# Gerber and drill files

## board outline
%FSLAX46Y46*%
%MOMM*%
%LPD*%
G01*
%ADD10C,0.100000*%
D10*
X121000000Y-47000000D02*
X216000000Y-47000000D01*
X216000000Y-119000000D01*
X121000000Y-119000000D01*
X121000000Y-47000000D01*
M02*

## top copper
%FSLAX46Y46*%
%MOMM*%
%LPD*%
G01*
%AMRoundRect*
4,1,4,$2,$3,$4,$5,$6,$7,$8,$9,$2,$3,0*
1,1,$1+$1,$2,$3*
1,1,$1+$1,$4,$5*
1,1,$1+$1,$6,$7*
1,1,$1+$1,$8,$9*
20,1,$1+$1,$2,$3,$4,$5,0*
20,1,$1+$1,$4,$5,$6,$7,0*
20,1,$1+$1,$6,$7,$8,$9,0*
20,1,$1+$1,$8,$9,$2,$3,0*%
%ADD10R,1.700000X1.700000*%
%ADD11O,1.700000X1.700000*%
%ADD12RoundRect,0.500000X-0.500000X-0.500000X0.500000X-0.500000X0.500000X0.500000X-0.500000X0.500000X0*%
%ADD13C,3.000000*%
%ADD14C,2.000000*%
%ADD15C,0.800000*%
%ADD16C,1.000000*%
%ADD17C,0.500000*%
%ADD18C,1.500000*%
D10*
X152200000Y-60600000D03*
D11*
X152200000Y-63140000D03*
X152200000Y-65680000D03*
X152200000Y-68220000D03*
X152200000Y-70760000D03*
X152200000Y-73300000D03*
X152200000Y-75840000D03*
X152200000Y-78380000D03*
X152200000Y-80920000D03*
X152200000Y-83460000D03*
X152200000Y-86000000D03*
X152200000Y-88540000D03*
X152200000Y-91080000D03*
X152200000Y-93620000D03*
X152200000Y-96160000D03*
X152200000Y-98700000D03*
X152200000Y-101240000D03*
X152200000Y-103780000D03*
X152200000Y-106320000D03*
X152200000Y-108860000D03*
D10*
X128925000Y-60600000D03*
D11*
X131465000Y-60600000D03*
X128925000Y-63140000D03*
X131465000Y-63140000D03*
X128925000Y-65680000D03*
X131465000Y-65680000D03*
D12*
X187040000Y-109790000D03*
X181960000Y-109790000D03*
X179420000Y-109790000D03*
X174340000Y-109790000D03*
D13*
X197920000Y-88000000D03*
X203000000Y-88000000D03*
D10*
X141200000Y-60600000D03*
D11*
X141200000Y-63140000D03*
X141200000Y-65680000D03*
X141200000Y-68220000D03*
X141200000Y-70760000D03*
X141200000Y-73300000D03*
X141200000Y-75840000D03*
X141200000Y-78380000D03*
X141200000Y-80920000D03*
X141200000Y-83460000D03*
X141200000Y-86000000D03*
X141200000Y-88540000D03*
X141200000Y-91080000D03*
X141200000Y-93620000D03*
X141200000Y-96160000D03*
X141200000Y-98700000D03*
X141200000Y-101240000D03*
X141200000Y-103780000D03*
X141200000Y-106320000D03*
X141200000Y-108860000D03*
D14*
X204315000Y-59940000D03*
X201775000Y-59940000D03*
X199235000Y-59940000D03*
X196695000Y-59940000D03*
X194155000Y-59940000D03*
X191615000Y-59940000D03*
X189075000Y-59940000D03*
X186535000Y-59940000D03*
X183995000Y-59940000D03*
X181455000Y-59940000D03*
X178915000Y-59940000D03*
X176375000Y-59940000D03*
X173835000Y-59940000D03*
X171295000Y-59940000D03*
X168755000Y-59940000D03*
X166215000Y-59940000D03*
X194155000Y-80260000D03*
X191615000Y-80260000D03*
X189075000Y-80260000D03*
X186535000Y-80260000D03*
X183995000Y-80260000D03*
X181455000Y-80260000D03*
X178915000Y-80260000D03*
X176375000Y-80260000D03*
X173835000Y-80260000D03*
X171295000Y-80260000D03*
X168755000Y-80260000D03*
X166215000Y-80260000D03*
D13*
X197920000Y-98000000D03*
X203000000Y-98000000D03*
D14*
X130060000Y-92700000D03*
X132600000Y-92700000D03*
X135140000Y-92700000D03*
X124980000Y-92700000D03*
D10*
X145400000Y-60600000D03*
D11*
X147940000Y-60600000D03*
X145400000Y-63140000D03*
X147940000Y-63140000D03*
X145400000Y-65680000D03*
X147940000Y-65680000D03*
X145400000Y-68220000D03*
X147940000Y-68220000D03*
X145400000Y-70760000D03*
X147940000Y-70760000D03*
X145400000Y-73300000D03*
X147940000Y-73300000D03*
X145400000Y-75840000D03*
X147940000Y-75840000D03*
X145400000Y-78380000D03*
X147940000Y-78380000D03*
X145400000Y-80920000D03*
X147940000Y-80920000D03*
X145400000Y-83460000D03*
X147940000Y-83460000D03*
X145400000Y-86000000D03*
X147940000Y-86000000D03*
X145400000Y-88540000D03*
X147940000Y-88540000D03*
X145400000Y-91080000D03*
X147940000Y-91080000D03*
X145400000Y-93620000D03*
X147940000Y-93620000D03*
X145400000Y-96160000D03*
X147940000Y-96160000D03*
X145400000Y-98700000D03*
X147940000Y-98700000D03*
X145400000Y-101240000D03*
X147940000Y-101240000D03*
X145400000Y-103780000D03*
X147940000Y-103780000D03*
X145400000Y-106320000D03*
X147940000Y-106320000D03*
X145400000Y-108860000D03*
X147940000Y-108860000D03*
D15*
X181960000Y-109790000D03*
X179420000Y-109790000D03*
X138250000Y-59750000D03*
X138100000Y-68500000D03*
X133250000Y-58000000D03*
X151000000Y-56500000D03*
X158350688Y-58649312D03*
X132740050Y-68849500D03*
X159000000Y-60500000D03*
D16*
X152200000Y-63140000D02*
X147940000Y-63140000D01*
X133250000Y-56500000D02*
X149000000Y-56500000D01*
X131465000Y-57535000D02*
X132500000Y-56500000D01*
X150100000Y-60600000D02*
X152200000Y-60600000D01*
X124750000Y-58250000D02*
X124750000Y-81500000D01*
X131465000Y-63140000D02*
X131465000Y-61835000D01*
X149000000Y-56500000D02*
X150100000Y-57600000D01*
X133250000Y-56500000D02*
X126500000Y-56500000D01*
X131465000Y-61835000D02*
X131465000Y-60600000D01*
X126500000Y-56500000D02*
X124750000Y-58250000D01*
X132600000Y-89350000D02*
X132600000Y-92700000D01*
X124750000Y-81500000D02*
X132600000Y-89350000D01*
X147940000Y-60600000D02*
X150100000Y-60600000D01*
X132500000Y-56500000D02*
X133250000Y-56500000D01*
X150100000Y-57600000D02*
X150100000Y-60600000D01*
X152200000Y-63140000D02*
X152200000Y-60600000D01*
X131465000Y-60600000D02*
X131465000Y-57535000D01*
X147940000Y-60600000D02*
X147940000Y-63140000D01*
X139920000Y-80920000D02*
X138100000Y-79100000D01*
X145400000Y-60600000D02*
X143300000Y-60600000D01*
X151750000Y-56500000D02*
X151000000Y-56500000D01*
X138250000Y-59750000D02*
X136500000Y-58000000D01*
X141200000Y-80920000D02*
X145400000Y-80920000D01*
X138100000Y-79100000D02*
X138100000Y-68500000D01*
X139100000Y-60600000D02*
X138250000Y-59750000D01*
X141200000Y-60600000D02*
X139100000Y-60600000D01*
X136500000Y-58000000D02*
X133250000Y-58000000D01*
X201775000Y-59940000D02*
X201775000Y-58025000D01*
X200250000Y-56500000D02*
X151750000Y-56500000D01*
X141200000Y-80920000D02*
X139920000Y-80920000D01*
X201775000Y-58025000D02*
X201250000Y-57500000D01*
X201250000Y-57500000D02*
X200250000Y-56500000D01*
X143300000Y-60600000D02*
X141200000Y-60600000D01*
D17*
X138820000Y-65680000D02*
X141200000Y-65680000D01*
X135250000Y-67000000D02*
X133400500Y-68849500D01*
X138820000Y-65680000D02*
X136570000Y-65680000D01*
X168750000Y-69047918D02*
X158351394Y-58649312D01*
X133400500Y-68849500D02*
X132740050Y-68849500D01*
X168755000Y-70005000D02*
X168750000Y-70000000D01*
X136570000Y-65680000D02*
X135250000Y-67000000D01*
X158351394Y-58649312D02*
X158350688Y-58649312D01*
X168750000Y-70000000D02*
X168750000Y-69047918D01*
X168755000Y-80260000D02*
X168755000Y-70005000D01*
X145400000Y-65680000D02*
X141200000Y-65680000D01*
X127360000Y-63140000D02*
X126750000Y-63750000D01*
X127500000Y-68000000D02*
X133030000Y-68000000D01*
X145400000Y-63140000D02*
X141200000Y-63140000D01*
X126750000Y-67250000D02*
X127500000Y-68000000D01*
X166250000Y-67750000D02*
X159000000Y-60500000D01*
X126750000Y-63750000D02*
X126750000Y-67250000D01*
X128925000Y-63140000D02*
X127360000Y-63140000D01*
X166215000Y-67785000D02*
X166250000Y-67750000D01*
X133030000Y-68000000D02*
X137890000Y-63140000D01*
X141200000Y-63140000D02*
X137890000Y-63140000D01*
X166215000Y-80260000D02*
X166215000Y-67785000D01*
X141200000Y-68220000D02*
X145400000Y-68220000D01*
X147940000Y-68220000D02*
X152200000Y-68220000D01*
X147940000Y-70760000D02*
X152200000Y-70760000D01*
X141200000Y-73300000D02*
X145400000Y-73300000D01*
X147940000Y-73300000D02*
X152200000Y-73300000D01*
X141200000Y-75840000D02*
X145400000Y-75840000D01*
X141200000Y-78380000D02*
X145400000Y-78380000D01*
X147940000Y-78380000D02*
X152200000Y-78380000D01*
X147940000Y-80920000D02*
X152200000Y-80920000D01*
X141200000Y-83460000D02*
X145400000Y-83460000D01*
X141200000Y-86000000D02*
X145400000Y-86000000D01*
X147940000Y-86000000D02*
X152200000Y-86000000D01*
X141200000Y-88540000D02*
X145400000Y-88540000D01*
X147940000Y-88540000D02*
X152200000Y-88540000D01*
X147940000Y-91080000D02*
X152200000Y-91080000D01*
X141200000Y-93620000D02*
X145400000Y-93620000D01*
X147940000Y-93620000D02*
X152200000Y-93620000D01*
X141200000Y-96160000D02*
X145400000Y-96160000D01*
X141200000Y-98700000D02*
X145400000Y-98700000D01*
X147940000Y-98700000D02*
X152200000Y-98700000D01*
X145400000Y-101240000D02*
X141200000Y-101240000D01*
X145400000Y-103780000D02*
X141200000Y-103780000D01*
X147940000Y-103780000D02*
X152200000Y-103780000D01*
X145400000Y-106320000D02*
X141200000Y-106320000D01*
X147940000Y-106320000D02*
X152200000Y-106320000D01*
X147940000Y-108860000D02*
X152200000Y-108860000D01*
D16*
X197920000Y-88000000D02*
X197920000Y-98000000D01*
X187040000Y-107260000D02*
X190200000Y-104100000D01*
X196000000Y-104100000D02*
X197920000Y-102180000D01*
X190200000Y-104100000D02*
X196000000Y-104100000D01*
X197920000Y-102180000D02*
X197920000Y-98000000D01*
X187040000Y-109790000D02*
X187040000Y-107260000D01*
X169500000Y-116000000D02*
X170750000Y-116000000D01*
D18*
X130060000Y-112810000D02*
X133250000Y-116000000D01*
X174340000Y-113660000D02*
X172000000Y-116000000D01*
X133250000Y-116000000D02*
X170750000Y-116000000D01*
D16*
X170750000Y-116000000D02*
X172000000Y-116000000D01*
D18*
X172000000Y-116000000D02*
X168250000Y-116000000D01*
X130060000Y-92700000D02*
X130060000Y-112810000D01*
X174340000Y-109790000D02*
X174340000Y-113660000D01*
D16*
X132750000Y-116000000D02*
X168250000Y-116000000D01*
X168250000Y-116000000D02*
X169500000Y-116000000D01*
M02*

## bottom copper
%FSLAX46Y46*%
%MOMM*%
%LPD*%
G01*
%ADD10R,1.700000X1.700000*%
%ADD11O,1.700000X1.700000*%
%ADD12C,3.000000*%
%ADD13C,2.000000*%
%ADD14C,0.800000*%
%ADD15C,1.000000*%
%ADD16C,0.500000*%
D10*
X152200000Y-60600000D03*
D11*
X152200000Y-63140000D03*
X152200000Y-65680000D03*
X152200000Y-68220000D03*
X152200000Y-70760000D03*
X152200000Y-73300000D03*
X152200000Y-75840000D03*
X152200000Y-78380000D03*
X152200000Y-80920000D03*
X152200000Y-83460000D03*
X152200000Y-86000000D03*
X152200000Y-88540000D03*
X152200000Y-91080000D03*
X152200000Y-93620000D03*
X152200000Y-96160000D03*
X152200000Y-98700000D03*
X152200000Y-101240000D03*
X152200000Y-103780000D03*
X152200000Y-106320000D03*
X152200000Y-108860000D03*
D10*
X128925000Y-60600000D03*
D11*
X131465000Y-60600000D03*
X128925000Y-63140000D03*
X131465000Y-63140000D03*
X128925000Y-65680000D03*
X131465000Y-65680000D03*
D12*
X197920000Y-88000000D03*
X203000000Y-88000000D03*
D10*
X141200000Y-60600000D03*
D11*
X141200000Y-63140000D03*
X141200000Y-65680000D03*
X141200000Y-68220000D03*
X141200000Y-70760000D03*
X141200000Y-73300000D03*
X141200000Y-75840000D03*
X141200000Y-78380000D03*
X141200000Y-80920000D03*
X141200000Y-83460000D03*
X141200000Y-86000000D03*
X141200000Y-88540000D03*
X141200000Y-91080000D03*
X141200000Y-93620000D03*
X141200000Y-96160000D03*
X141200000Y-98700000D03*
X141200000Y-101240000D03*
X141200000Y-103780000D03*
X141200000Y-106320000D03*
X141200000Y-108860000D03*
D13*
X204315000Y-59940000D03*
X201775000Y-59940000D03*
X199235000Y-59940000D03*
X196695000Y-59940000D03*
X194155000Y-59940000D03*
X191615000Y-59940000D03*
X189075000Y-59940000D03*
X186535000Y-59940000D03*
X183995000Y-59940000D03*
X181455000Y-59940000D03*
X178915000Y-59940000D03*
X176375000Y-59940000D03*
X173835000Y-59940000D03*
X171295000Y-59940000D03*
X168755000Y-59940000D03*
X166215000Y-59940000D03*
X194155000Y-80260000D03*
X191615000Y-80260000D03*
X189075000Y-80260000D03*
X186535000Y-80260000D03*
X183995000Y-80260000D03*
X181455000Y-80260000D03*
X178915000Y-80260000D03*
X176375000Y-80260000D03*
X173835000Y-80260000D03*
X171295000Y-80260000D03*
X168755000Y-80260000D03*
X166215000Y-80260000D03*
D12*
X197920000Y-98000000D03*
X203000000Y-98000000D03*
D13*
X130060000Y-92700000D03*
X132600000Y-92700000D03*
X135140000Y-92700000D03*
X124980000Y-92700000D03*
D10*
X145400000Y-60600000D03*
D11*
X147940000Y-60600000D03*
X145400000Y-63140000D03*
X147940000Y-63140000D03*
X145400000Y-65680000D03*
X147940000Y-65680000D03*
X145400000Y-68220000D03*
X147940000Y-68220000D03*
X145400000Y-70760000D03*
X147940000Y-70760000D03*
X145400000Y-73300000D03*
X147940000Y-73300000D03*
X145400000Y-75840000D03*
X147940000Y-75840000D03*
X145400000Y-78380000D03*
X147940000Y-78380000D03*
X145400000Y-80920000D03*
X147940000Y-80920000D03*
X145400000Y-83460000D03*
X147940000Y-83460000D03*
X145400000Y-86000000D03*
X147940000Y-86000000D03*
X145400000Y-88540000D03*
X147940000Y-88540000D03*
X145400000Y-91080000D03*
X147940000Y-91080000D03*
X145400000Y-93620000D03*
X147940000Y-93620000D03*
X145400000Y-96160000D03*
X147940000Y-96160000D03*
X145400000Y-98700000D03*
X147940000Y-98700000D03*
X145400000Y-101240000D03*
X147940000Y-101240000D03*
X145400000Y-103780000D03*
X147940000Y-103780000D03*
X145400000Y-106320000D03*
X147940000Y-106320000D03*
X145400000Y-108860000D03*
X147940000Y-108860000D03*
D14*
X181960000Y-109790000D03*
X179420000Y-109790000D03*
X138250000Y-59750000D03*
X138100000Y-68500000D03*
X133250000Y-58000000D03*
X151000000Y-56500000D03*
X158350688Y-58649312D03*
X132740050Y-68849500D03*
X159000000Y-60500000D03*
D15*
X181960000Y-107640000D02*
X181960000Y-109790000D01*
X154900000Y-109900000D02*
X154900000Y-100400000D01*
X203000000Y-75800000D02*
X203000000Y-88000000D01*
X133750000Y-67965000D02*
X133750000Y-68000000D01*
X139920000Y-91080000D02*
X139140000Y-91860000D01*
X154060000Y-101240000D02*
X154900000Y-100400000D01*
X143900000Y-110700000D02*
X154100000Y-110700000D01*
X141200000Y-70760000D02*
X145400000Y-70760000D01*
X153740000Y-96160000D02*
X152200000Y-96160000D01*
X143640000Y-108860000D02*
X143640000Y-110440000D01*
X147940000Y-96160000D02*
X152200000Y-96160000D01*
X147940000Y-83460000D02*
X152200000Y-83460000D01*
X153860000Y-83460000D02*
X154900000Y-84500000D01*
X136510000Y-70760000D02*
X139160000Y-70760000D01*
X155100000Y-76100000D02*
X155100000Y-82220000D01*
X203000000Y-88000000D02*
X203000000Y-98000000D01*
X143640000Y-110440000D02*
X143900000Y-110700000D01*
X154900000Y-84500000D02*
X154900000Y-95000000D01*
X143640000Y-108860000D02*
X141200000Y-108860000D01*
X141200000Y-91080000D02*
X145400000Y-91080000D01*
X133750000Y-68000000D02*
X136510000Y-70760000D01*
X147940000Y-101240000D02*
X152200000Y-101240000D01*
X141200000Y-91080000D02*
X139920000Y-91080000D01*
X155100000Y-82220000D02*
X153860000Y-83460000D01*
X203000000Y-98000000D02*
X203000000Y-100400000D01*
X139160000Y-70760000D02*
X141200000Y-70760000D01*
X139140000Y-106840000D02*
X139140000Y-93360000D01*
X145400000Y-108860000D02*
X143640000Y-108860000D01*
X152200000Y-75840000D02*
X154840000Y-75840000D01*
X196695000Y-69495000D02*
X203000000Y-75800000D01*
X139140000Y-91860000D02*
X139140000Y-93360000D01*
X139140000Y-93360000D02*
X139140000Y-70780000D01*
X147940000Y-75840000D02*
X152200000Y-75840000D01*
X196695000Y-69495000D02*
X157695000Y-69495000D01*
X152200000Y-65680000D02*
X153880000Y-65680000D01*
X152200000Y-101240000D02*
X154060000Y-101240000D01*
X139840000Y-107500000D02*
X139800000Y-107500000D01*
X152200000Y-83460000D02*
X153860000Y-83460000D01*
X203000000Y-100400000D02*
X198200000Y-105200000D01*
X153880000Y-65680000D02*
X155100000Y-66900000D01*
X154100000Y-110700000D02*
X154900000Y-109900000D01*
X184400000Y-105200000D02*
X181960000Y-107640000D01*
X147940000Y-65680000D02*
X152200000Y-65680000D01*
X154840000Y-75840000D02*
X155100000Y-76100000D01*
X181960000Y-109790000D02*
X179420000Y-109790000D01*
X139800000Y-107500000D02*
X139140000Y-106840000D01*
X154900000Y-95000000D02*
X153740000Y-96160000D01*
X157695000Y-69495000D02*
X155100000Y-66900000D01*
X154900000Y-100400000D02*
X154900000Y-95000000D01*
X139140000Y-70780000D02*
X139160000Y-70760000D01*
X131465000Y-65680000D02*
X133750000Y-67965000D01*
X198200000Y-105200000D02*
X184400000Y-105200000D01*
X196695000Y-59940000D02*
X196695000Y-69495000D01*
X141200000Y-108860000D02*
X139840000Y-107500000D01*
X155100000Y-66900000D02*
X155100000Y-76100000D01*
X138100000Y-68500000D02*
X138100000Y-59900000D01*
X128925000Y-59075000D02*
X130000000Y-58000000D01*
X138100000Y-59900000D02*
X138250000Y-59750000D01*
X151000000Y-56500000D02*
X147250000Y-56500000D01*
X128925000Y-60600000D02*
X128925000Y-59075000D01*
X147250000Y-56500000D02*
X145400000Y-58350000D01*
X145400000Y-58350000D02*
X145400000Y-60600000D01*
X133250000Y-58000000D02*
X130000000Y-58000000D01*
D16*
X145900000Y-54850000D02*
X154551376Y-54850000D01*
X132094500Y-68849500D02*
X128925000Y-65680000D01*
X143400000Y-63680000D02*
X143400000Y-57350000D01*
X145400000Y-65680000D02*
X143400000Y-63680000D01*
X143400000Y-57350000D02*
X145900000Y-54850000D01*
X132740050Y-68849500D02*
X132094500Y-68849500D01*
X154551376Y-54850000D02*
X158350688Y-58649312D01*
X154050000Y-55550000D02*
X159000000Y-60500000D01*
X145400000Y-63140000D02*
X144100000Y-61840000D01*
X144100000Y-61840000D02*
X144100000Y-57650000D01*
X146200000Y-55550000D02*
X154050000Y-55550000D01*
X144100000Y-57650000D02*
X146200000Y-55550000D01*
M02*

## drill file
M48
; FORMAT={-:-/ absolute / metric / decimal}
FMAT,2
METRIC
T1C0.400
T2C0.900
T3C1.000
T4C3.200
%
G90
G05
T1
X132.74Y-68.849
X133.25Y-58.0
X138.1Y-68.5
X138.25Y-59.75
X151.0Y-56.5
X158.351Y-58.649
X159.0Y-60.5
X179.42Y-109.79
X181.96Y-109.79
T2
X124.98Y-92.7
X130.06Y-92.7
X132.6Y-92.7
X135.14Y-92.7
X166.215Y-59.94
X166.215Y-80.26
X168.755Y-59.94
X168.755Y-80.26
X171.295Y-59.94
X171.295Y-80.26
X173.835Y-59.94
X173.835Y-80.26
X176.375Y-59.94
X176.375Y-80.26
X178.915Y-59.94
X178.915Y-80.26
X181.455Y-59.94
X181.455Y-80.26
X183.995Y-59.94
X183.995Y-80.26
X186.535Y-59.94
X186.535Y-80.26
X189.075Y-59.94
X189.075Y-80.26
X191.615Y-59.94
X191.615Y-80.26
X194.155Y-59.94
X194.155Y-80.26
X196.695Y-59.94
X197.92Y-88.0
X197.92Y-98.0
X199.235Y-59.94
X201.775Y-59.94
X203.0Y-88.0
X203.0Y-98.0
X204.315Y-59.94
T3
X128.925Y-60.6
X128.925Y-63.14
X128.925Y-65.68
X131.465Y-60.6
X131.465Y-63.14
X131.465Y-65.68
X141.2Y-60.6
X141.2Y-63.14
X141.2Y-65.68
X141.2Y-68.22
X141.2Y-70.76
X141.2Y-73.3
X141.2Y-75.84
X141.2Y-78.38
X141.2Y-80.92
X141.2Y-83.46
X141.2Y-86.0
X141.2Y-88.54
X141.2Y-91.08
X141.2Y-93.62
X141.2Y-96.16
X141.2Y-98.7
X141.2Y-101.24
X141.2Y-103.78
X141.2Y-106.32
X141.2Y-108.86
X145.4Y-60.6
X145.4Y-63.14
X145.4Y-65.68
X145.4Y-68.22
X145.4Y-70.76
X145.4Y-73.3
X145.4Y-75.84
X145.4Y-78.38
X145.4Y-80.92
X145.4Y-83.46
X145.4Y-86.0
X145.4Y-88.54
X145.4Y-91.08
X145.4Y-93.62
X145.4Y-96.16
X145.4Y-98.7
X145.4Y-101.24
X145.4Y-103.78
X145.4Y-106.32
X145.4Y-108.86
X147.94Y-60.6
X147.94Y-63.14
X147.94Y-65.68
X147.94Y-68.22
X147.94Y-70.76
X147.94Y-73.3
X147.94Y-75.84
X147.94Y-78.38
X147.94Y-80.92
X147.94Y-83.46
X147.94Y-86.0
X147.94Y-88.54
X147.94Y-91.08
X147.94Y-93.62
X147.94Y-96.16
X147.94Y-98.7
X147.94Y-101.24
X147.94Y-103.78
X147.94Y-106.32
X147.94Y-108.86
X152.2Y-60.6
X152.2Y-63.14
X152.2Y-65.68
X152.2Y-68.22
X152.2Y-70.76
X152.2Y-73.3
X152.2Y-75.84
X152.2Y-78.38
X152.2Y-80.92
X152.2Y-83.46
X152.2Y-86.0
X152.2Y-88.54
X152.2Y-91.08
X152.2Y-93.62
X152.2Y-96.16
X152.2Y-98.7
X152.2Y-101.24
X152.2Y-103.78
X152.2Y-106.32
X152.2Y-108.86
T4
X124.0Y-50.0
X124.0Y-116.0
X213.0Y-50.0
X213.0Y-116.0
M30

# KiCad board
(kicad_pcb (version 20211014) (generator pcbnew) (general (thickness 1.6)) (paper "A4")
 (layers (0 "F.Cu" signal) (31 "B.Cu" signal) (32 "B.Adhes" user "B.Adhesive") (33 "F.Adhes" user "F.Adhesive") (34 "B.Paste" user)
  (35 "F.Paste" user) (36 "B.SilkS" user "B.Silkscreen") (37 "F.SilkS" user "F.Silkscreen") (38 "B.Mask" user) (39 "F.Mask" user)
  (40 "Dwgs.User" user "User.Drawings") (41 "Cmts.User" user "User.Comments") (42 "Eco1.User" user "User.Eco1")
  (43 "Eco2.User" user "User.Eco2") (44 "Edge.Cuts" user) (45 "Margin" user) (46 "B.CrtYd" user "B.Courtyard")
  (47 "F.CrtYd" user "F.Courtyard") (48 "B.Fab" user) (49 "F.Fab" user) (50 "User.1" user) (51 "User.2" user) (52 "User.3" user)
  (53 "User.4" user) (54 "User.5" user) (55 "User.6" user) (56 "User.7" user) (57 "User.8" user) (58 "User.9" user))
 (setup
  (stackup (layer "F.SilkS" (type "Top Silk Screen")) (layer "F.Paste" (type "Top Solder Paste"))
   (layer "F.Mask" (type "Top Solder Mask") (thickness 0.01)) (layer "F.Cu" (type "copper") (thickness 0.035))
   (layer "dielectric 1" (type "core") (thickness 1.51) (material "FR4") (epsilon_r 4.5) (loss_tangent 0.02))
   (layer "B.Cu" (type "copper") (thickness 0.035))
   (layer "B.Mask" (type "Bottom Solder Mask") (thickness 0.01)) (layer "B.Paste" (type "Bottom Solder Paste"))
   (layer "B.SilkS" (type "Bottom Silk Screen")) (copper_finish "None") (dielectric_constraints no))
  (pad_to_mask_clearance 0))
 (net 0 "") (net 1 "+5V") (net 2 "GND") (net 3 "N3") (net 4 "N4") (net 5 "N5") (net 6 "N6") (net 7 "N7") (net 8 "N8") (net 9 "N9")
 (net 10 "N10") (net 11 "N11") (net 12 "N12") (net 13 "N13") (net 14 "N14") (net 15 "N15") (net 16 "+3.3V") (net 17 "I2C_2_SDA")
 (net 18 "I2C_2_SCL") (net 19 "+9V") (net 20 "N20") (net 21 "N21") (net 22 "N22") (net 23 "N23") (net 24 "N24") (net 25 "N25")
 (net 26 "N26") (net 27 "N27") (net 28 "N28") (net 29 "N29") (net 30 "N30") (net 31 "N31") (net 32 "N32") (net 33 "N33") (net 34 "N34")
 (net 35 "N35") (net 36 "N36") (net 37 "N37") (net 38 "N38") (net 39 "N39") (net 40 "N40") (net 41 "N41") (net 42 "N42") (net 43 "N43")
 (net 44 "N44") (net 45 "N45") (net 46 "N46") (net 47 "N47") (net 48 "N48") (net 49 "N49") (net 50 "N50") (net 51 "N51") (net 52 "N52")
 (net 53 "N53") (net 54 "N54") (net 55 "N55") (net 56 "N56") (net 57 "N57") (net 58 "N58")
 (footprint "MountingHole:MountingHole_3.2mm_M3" (layer "F.Cu") (at 213 50)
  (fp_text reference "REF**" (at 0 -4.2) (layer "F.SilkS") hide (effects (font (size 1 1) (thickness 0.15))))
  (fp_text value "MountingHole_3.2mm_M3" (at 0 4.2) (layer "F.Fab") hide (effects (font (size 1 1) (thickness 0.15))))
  (pad "" np_thru_hole circle (at 0 0) (size 3.2 3.2) (drill 3.2) (layers F&B.Cu *.Mask)))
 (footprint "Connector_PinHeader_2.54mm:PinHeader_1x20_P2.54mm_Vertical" (layer "F.Cu") (at 152.2 60.6)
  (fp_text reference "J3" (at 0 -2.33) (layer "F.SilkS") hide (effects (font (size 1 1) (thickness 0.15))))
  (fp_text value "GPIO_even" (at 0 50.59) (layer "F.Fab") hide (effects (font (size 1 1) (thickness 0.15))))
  (pad "1" thru_hole rect (at 0 0) (size 1.7 1.7) (drill 1) (layers *.Cu *.Mask) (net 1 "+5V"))
  (pad "2" thru_hole oval (at 0 2.54) (size 1.7 1.7) (drill 1) (layers *.Cu *.Mask) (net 1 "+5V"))
  (pad "3" thru_hole oval (at 0 5.08) (size 1.7 1.7) (drill 1) (layers *.Cu *.Mask) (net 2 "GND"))
  (pad "4" thru_hole oval (at 0 7.62) (size 1.7 1.7) (drill 1) (layers *.Cu *.Mask) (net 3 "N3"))
  (pad "5" thru_hole oval (at 0 10.16) (size 1.7 1.7) (drill 1) (layers *.Cu *.Mask) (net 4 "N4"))
  (pad "6" thru_hole oval (at 0 12.7) (size 1.7 1.7) (drill 1) (layers *.Cu *.Mask) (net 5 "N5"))
  (pad "7" thru_hole oval (at 0 15.24) (size 1.7 1.7) (drill 1) (layers *.Cu *.Mask) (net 2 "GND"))
  (pad "8" thru_hole oval (at 0 17.78) (size 1.7 1.7) (drill 1) (layers *.Cu *.Mask) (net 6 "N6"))
  (pad "9" thru_hole oval (at 0 20.32) (size 1.7 1.7) (drill 1) (layers *.Cu *.Mask) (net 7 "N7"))
  (pad "10" thru_hole oval (at 0 22.86) (size 1.7 1.7) (drill 1) (layers *.Cu *.Mask) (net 2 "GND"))
  (pad "11" thru_hole oval (at 0 25.4) (size 1.7 1.7) (drill 1) (layers *.Cu *.Mask) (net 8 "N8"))
  (pad "12" thru_hole oval (at 0 27.94) (size 1.7 1.7) (drill 1) (layers *.Cu *.Mask) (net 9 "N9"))
  (pad "13" thru_hole oval (at 0 30.48) (size 1.7 1.7) (drill 1) (layers *.Cu *.Mask) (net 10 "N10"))
  (pad "14" thru_hole oval (at 0 33.02) (size 1.7 1.7) (drill 1) (layers *.Cu *.Mask) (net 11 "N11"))
  (pad "15" thru_hole oval (at 0 35.56) (size 1.7 1.7) (drill 1) (layers *.Cu *.Mask) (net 2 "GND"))
  (pad "16" thru_hole oval (at 0 38.1) (size 1.7 1.7) (drill 1) (layers *.Cu *.Mask) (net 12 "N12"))
  (pad "17" thru_hole oval (at 0 40.64) (size 1.7 1.7) (drill 1) (layers *.Cu *.Mask) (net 2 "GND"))
  (pad "18" thru_hole oval (at 0 43.18) (size 1.7 1.7) (drill 1) (layers *.Cu *.Mask) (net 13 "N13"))
  (pad "19" thru_hole oval (at 0 45.72) (size 1.7 1.7) (drill 1) (layers *.Cu *.Mask) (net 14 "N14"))
  (pad "20" thru_hole oval (at 0 48.26) (size 1.7 1.7) (drill 1) (layers *.Cu *.Mask) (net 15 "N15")))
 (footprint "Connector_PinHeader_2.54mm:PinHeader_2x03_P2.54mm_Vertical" (layer "F.Cu") (at 128.925 60.6)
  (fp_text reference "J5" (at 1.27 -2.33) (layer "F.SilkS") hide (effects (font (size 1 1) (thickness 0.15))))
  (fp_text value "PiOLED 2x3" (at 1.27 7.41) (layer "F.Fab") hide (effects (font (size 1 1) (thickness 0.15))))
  (pad "1" thru_hole rect (at 0 0) (size 1.7 1.7) (drill 1) (layers *.Cu *.Mask) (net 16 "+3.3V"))
  (pad "2" thru_hole oval (at 2.54 0) (size 1.7 1.7) (drill 1) (layers *.Cu *.Mask) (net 1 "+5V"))
  (pad "3" thru_hole oval (at 0 2.54) (size 1.7 1.7) (drill 1) (layers *.Cu *.Mask) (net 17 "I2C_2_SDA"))
  (pad "4" thru_hole oval (at 2.54 2.54) (size 1.7 1.7) (drill 1) (layers *.Cu *.Mask) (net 1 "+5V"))
  (pad "5" thru_hole oval (at 0 5.08) (size 1.7 1.7) (drill 1) (layers *.Cu *.Mask) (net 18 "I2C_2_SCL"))
  (pad "6" thru_hole oval (at 2.54 5.08) (size 1.7 1.7) (drill 1) (layers *.Cu *.Mask) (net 2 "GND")))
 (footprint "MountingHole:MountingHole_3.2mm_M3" (layer "F.Cu") (at 124 50)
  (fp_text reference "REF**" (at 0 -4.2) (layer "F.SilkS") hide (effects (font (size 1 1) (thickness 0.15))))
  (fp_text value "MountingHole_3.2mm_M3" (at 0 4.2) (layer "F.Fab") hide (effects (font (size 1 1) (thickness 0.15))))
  (pad "" np_thru_hole circle (at 0 0) (size 3.2 3.2) (drill 3.2) (layers F&B.Cu *.Mask)))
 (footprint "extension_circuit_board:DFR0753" (layer "F.Cu") (at 176.5 98.87)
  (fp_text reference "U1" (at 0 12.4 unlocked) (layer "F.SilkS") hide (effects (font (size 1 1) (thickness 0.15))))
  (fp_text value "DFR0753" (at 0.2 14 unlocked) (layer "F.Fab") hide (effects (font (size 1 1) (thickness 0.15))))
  (pad "1" smd roundrect (at 10.54 10.92) (size 2 2) (layers "F.Cu" "F.Paste" "F.Mask") (roundrect_rratio 0.25) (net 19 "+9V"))
  (pad "2" smd roundrect (at 5.46 10.92) (size 2 2) (layers "F.Cu" "F.Paste" "F.Mask") (roundrect_rratio 0.25) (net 2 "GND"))
  (pad "3" smd roundrect (at 2.92 10.92) (size 2 2) (layers "F.Cu" "F.Paste" "F.Mask") (roundrect_rratio 0.25) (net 2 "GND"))
  (pad "4" smd roundrect (at -2.16 10.92) (size 2 2) (layers "F.Cu" "F.Paste" "F.Mask") (roundrect_rratio 0.25) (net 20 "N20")))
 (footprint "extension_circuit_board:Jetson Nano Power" (layer "F.Cu") (at 200.46 90.54)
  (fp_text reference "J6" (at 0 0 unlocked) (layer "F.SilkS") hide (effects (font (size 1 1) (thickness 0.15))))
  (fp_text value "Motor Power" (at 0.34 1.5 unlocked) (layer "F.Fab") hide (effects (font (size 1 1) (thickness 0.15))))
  (pad "1" thru_hole circle (at -2.54 -2.54) (size 3 3) (drill 0.9) (layers *.Cu *.Mask) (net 19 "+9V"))
  (pad "2" thru_hole circle (at 2.54 -2.54) (size 3 3) (drill 0.9) (layers *.Cu *.Mask) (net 2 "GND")))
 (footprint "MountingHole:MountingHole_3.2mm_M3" (layer "F.Cu") (at 124 116)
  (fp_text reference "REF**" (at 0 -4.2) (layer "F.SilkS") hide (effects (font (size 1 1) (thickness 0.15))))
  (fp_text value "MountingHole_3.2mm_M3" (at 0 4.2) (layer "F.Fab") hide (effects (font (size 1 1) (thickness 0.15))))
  (pad "" np_thru_hole circle (at 0 0) (size 3.2 3.2) (drill 3.2) (layers *.Cu *.Mask)))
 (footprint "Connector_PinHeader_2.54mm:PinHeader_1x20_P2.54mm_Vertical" (layer "F.Cu") (at 141.2 60.6)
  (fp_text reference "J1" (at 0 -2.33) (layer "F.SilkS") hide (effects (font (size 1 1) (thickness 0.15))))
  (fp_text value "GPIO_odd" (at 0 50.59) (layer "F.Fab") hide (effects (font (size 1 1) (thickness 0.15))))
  (pad "1" thru_hole rect (at 0 0) (size 1.7 1.7) (drill 1) (layers *.Cu *.Mask) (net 16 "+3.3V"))
  (pad "2" thru_hole oval (at 0 2.54) (size 1.7 1.7) (drill 1) (layers *.Cu *.Mask) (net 17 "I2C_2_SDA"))
  (pad "3" thru_hole oval (at 0 5.08) (size 1.7 1.7) (drill 1) (layers *.Cu *.Mask) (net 18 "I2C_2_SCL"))
  (pad "4" thru_hole oval (at 0 7.62) (size 1.7 1.7) (drill 1) (layers *.Cu *.Mask) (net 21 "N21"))
  (pad "5" thru_hole oval (at 0 10.16) (size 1.7 1.7) (drill 1) (layers *.Cu *.Mask) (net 2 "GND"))
  (pad "6" thru_hole oval (at 0 12.7) (size 1.7 1.7) (drill 1) (layers *.Cu *.Mask) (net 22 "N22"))
  (pad "7" thru_hole oval (at 0 15.24) (size 1.7 1.7) (drill 1) (layers *.Cu *.Mask) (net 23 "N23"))
  (pad "8" thru_hole oval (at 0 17.78) (size 1.7 1.7) (drill 1) (layers *.Cu *.Mask) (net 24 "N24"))
  (pad "9" thru_hole oval (at 0 20.32) (size 1.7 1.7) (drill 1) (layers *.Cu *.Mask) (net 16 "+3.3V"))
  (pad "10" thru_hole oval (at 0 22.86) (size 1.7 1.7) (drill 1) (layers *.Cu *.Mask) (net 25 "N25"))
  (pad "11" thru_hole oval (at 0 25.4) (size 1.7 1.7) (drill 1) (layers *.Cu *.Mask) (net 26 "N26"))
  (pad "12" thru_hole oval (at 0 27.94) (size 1.7 1.7) (drill 1) (layers *.Cu *.Mask) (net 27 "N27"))
  (pad "13" thru_hole oval (at 0 30.48) (size 1.7 1.7) (drill 1) (layers *.Cu *.Mask) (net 2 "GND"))
  (pad "14" thru_hole oval (at 0 33.02) (size 1.7 1.7) (drill 1) (layers *.Cu *.Mask) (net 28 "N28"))
  (pad "15" thru_hole oval (at 0 35.56) (size 1.7 1.7) (drill 1) (layers *.Cu *.Mask) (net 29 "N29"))
  (pad "16" thru_hole oval (at 0 38.1) (size 1.7 1.7) (drill 1) (layers *.Cu *.Mask) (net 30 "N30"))
  (pad "17" thru_hole oval (at 0 40.64) (size 1.7 1.7) (drill 1) (layers *.Cu *.Mask) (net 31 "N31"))
  (pad "18" thru_hole oval (at 0 43.18) (size 1.7 1.7) (drill 1) (layers *.Cu *.Mask) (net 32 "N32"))
  (pad "19" thru_hole oval (at 0 45.72) (size 1.7 1.7) (drill 1) (layers *.Cu *.Mask) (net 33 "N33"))
  (pad "20" thru_hole oval (at 0 48.26) (size 1.7 1.7) (drill 1) (layers *.Cu *.Mask) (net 2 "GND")))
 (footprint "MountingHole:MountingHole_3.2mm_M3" (layer "F.Cu") (at 213 116)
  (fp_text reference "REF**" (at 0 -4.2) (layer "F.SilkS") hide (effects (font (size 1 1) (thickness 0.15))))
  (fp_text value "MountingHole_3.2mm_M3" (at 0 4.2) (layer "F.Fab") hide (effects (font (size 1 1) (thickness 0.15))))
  (pad "" np_thru_hole circle (at 0 0) (size 3.2 3.2) (drill 3.2) (layers F&B.Cu *.Mask)))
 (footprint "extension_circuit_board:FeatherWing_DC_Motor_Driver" (layer "F.Cu") (at 157.325 71.37 -90)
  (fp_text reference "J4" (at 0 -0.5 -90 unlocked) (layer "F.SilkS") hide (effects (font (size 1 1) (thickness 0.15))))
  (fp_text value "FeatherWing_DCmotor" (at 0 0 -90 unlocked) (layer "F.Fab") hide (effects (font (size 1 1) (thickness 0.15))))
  (pad "1" thru_hole circle (at -11.43 -46.99 270) (size 2 2) (drill 0.9) (layers *.Cu *.Mask) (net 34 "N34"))
  (pad "2" thru_hole circle (at -11.43 -44.45 270) (size 2 2) (drill 0.9) (layers *.Cu *.Mask) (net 16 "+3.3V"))
  (pad "3" thru_hole circle (at -11.43 -41.91 270) (size 2 2) (drill 0.9) (layers *.Cu *.Mask) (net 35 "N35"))
  (pad "4" thru_hole circle (at -11.43 -39.37 270) (size 2 2) (drill 0.9) (layers *.Cu *.Mask) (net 2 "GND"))
  (pad "5" thru_hole circle (at -11.43 -36.83 270) (size 2 2) (drill 0.9) (layers *.Cu *.Mask) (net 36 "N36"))
  (pad "6" thru_hole circle (at -11.43 -34.29 270) (size 2 2) (drill 0.9) (layers *.Cu *.Mask) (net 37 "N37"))
  (pad "7" thru_hole circle (at -11.43 -31.75 270) (size 2 2) (drill 0.9) (layers *.Cu *.Mask) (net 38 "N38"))
  (pad "8" thru_hole circle (at -11.43 -29.21 270) (size 2 2) (drill 0.9) (layers *.Cu *.Mask) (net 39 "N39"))
  (pad "9" thru_hole circle (at -11.43 -26.67 270) (size 2 2) (drill 0.9) (layers *.Cu *.Mask) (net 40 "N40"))
  (pad "10" thru_hole circle (at -11.43 -24.13 270) (size 2 2) (drill 0.9) (layers *.Cu *.Mask) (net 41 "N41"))
  (pad "11" thru_hole circle (at -11.43 -21.59 270) (size 2 2) (drill 0.9) (layers *.Cu *.Mask) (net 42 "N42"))
  (pad "12" thru_hole circle (at -11.43 -19.05 270) (size 2 2) (drill 0.9) (layers *.Cu *.Mask) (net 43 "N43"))
  (pad "13" thru_hole circle (at -11.43 -16.51 270) (size 2 2) (drill 0.9) (layers *.Cu *.Mask) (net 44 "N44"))
  (pad "14" thru_hole circle (at -11.43 -13.97 270) (size 2 2) (drill 0.9) (layers *.Cu *.Mask) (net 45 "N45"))
  (pad "15" thru_hole circle (at -11.43 -11.43 270) (size 2 2) (drill 0.9) (layers *.Cu *.Mask) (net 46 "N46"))
  (pad "16" thru_hole circle (at -11.43 -8.89 270) (size 2 2) (drill 0.9) (layers *.Cu *.Mask) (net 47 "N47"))
  (pad "21" thru_hole circle (at 8.89 -36.83 270) (size 2 2) (drill 0.9) (layers *.Cu *.Mask) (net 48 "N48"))
  (pad "22" thru_hole circle (at 8.89 -34.29 270) (size 2 2) (drill 0.9) (layers *.Cu *.Mask) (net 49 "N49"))
  (pad "23" thru_hole circle (at 8.89 -31.75 270) (size 2 2) (drill 0.9) (layers *.Cu *.Mask) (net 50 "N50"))
  (pad "24" thru_hole circle (at 8.89 -29.21 270) (size 2 2) (drill 0.9) (layers *.Cu *.Mask) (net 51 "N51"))
  (pad "25" thru_hole circle (at 8.89 -26.67 270) (size 2 2) (drill 0.9) (layers *.Cu *.Mask) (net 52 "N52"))
  (pad "26" thru_hole circle (at 8.89 -24.13 270) (size 2 2) (drill 0.9) (layers *.Cu *.Mask) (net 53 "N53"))
  (pad "27" thru_hole circle (at 8.89 -21.59 270) (size 2 2) (drill 0.9) (layers *.Cu *.Mask) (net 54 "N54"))
  (pad "28" thru_hole circle (at 8.89 -19.05 270) (size 2 2) (drill 0.9) (layers *.Cu *.Mask) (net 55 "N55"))
  (pad "29" thru_hole circle (at 8.89 -16.51 270) (size 2 2) (drill 0.9) (layers *.Cu *.Mask) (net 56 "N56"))
  (pad "30" thru_hole circle (at 8.89 -13.97 270) (size 2 2) (drill 0.9) (layers *.Cu *.Mask) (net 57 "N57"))
  (pad "31" thru_hole circle (at 8.89 -11.43 270) (size 2 2) (drill 0.9) (layers *.Cu *.Mask) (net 18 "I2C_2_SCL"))
  (pad "32" thru_hole circle (at 8.89 -8.89 270) (size 2 2) (drill 0.9) (layers *.Cu *.Mask) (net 17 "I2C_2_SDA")))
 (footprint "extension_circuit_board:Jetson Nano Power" (layer "F.Cu") (at 200.46 100.54)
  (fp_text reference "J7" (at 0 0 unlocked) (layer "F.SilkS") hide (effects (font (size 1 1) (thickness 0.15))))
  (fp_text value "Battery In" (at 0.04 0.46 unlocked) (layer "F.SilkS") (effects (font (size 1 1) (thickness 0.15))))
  (pad "1" thru_hole circle (at -2.54 -2.54) (size 3 3) (drill 0.9) (layers *.Cu *.Mask) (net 19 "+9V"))
  (pad "2" thru_hole circle (at 2.54 -2.54) (size 3 3) (drill 0.9) (layers *.Cu *.Mask) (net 2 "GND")))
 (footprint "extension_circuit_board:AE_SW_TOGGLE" (layer "F.Cu") (at 122.44 92.7 -90)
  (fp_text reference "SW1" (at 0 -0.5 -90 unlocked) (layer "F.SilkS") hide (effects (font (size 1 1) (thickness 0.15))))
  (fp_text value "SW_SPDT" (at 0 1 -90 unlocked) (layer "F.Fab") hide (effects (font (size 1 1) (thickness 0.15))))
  (pad "1" thru_hole circle (at 0 -7.62 270) (size 2 2) (drill 0.9) (layers *.Cu *.Mask) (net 20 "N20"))
  (pad "2" thru_hole circle (at 0 -10.16 270) (size 2 2) (drill 0.9) (layers *.Cu *.Mask) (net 1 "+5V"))
  (pad "3" thru_hole circle (at 0 -12.7 270) (size 2 2) (drill 0.9) (layers *.Cu *.Mask) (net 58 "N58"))
  (pad "4" thru_hole circle (at 0 -2.54 270) (size 2 2) (drill 0.9) (layers *.Cu *.Mask)))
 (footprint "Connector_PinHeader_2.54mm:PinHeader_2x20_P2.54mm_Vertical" (layer "F.Cu") (at 145.4 60.6)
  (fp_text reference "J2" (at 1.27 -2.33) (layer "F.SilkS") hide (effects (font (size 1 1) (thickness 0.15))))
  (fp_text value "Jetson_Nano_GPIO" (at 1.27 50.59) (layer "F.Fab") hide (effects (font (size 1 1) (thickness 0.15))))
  (pad "1" thru_hole rect (at 0 0) (size 1.7 1.7) (drill 1) (layers *.Cu *.Mask) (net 16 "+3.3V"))
  (pad "2" thru_hole oval (at 2.54 0) (size 1.7 1.7) (drill 1) (layers *.Cu *.Mask) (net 1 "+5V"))
  (pad "3" thru_hole oval (at 0 2.54) (size 1.7 1.7) (drill 1) (layers *.Cu *.Mask) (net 17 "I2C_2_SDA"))
  (pad "4" thru_hole oval (at 2.54 2.54) (size 1.7 1.7) (drill 1) (layers *.Cu *.Mask) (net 1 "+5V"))
  (pad "5" thru_hole oval (at 0 5.08) (size 1.7 1.7) (drill 1) (layers *.Cu *.Mask) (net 18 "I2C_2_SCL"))
  (pad "6" thru_hole oval (at 2.54 5.08) (size 1.7 1.7) (drill 1) (layers *.Cu *.Mask) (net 2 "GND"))
  (pad "7" thru_hole oval (at 0 7.62) (size 1.7 1.7) (drill 1) (layers *.Cu *.Mask) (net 21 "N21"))
  (pad "8" thru_hole oval (at 2.54 7.62) (size 1.7 1.7) (drill 1) (layers *.Cu *.Mask) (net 3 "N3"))
  (pad "9" thru_hole oval (at 0 10.16) (size 1.7 1.7) (drill 1) (layers *.Cu *.Mask) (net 2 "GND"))
  (pad "10" thru_hole oval (at 2.54 10.16) (size 1.7 1.7) (drill 1) (layers *.Cu *.Mask) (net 4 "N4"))
  (pad "11" thru_hole oval (at 0 12.7) (size 1.7 1.7) (drill 1) (layers *.Cu *.Mask) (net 22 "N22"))
  (pad "12" thru_hole oval (at 2.54 12.7) (size 1.7 1.7) (drill 1) (layers *.Cu *.Mask) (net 5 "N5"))
  (pad "13" thru_hole oval (at 0 15.24) (size 1.7 1.7) (drill 1) (layers *.Cu *.Mask) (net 23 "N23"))
  (pad "14" thru_hole oval (at 2.54 15.24) (size 1.7 1.7) (drill 1) (layers *.Cu *.Mask) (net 2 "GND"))
  (pad "15" thru_hole oval (at 0 17.78) (size 1.7 1.7) (drill 1) (layers *.Cu *.Mask) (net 24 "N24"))
  (pad "16" thru_hole oval (at 2.54 17.78) (size 1.7 1.7) (drill 1) (layers *.Cu *.Mask) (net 6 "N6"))
  (pad "17" thru_hole oval (at 0 20.32) (size 1.7 1.7) (drill 1) (layers *.Cu *.Mask) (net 16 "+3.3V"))
  (pad "18" thru_hole oval (at 2.54 20.32) (size 1.7 1.7) (drill 1) (layers *.Cu *.Mask) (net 7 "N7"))
  (pad "19" thru_hole oval (at 0 22.86) (size 1.7 1.7) (drill 1) (layers *.Cu *.Mask) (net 25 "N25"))
  (pad "20" thru_hole oval (at 2.54 22.86) (size 1.7 1.7) (drill 1) (layers *.Cu *.Mask) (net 2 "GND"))
  (pad "21" thru_hole oval (at 0 25.4) (size 1.7 1.7) (drill 1) (layers *.Cu *.Mask) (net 26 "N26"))
  (pad "22" thru_hole oval (at 2.54 25.4) (size 1.7 1.7) (drill 1) (layers *.Cu *.Mask) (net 8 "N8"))
  (pad "23" thru_hole oval (at 0 27.94) (size 1.7 1.7) (drill 1) (layers *.Cu *.Mask) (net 27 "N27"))
  (pad "24" thru_hole oval (at 2.54 27.94) (size 1.7 1.7) (drill 1) (layers *.Cu *.Mask) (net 9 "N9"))
  (pad "25" thru_hole oval (at 0 30.48) (size 1.7 1.7) (drill 1) (layers *.Cu *.Mask) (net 2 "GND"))
  (pad "26" thru_hole oval (at 2.54 30.48) (size 1.7 1.7) (drill 1) (layers *.Cu *.Mask) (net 10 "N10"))
  (pad "27" thru_hole oval (at 0 33.02) (size 1.7 1.7) (drill 1) (layers *.Cu *.Mask) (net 28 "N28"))
  (pad "28" thru_hole oval (at 2.54 33.02) (size 1.7 1.7) (drill 1) (layers *.Cu *.Mask) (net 11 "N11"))
  (pad "29" thru_hole oval (at 0 35.56) (size 1.7 1.7) (drill 1) (layers *.Cu *.Mask) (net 29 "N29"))
  (pad "30" thru_hole oval (at 2.54 35.56) (size 1.7 1.7) (drill 1) (layers *.Cu *.Mask) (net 2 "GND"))
  (pad "31" thru_hole oval (at 0 38.1) (size 1.7 1.7) (drill 1) (layers *.Cu *.Mask) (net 30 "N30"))
  (pad "32" thru_hole oval (at 2.54 38.1) (size 1.7 1.7) (drill 1) (layers *.Cu *.Mask) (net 12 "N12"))
  (pad "33" thru_hole oval (at 0 40.64) (size 1.7 1.7) (drill 1) (layers *.Cu *.Mask) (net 31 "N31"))
  (pad "34" thru_hole oval (at 2.54 40.64) (size 1.7 1.7) (drill 1) (layers *.Cu *.Mask) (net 2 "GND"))
  (pad "35" thru_hole oval (at 0 43.18) (size 1.7 1.7) (drill 1) (layers *.Cu *.Mask) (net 32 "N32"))
  (pad "36" thru_hole oval (at 2.54 43.18) (size 1.7 1.7) (drill 1) (layers *.Cu *.Mask) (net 13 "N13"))
  (pad "37" thru_hole oval (at 0 45.72) (size 1.7 1.7) (drill 1) (layers *.Cu *.Mask) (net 33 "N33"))
  (pad "38" thru_hole oval (at 2.54 45.72) (size 1.7 1.7) (drill 1) (layers *.Cu *.Mask) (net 14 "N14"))
  (pad "39" thru_hole oval (at 0 48.26) (size 1.7 1.7) (drill 1) (layers *.Cu *.Mask) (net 2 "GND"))
  (pad "40" thru_hole oval (at 2.54 48.26) (size 1.7 1.7) (drill 1) (layers *.Cu *.Mask) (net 15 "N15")))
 (gr_rect (start 121 47) (end 216 119) (layer "Edge.Cuts") (width 0.1) (fill none))
 (segment (start 152.2 63.14) (end 147.94 63.14) (width 1) (layer "F.Cu") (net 1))
 (segment (start 133.25 56.5) (end 149 56.5) (width 1) (layer "F.Cu") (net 1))
 (segment (start 131.465 57.535) (end 132.5 56.5) (width 1) (layer "F.Cu") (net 1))
 (segment (start 150.1 60.6) (end 152.2 60.6) (width 1) (layer "F.Cu") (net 1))
 (segment (start 124.75 58.25) (end 124.75 81.5) (width 1) (layer "F.Cu") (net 1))
 (segment (start 131.465 63.14) (end 131.465 61.835) (width 1) (layer "F.Cu") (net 1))
 (segment (start 149 56.5) (end 150.1 57.6) (width 1) (layer "F.Cu") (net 1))
 (segment (start 133.25 56.5) (end 126.5 56.5) (width 1) (layer "F.Cu") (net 1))
 (segment (start 131.465 61.835) (end 131.465 60.6) (width 1) (layer "F.Cu") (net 1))
 (segment (start 126.5 56.5) (end 124.75 58.25) (width 1) (layer "F.Cu") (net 1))
 (segment (start 132.6 89.35) (end 132.6 92.7) (width 1) (layer "F.Cu") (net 1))
 (segment (start 124.75 81.5) (end 132.6 89.35) (width 1) (layer "F.Cu") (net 1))
 (segment (start 147.94 60.6) (end 150.1 60.6) (width 1) (layer "F.Cu") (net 1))
 (segment (start 132.5 56.5) (end 133.25 56.5) (width 1) (layer "F.Cu") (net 1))
 (segment (start 150.1 57.6) (end 150.1 60.6) (width 1) (layer "F.Cu") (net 1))
 (segment (start 152.2 63.14) (end 152.2 60.6) (width 1) (layer "F.Cu") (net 1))
 (segment (start 131.465 60.6) (end 131.465 57.535) (width 1) (layer "F.Cu") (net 1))
 (segment (start 147.94 60.6) (end 147.94 63.14) (width 1) (layer "F.Cu") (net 1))
 (via (at 181.96 109.79) (size 0.8) (drill 0.4) (layers "F.Cu" "B.Cu") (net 2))
 (via (at 179.42 109.79) (size 0.8) (drill 0.4) (layers "F.Cu" "B.Cu") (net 2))
 (segment (start 181.96 107.64) (end 181.96 109.79) (width 1) (layer "B.Cu") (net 2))
 (segment (start 154.9 109.9) (end 154.9 100.4) (width 1) (layer "B.Cu") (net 2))
 (segment (start 203 75.8) (end 203 88) (width 1) (layer "B.Cu") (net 2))
 (segment (start 133.75 67.965) (end 133.75 68) (width 1) (layer "B.Cu") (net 2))
 (segment (start 139.92 91.08) (end 139.14 91.86) (width 1) (layer "B.Cu") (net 2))
 (segment (start 154.06 101.24) (end 154.9 100.4) (width 1) (layer "B.Cu") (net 2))
 (segment (start 143.9 110.7) (end 154.1 110.7) (width 1) (layer "B.Cu") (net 2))
 (segment (start 141.2 70.76) (end 145.4 70.76) (width 1) (layer "B.Cu") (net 2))
 (segment (start 153.74 96.16) (end 152.2 96.16) (width 1) (layer "B.Cu") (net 2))
 (segment (start 143.64 108.86) (end 143.64 110.44) (width 1) (layer "B.Cu") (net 2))
 (segment (start 147.94 96.16) (end 152.2 96.16) (width 1) (layer "B.Cu") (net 2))
 (segment (start 147.94 83.46) (end 152.2 83.46) (width 1) (layer "B.Cu") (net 2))
 (segment (start 153.86 83.46) (end 154.9 84.5) (width 1) (layer "B.Cu") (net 2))
 (segment (start 136.51 70.76) (end 139.16 70.76) (width 1) (layer "B.Cu") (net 2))
 (segment (start 155.1 76.1) (end 155.1 82.22) (width 1) (layer "B.Cu") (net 2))
 (segment (start 203 88) (end 203 98) (width 1) (layer "B.Cu") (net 2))
 (segment (start 143.64 110.44) (end 143.9 110.7) (width 1) (layer "B.Cu") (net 2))
 (segment (start 154.9 84.5) (end 154.9 95) (width 1) (layer "B.Cu") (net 2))
 (segment (start 143.64 108.86) (end 141.2 108.86) (width 1) (layer "B.Cu") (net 2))
 (segment (start 141.2 91.08) (end 145.4 91.08) (width 1) (layer "B.Cu") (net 2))
 (segment (start 133.75 68) (end 136.51 70.76) (width 1) (layer "B.Cu") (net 2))
 (segment (start 147.94 101.24) (end 152.2 101.24) (width 1) (layer "B.Cu") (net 2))
 (segment (start 141.2 91.08) (end 139.92 91.08) (width 1) (layer "B.Cu") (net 2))
 (segment (start 155.1 82.22) (end 153.86 83.46) (width 1) (layer "B.Cu") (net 2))
 (segment (start 203 98) (end 203 100.4) (width 1) (layer "B.Cu") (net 2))
 (segment (start 139.16 70.76) (end 141.2 70.76) (width 1) (layer "B.Cu") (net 2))
 (segment (start 139.14 106.84) (end 139.14 93.36) (width 1) (layer "B.Cu") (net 2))
 (segment (start 145.4 108.86) (end 143.64 108.86) (width 1) (layer "B.Cu") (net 2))
 (segment (start 152.2 75.84) (end 154.84 75.84) (width 1) (layer "B.Cu") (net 2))
 (segment (start 196.695 69.495) (end 203 75.8) (width 1) (layer "B.Cu") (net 2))
 (segment (start 139.14 91.86) (end 139.14 93.36) (width 1) (layer "B.Cu") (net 2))
 (segment (start 139.14 93.36) (end 139.14 70.78) (width 1) (layer "B.Cu") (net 2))
 (segment (start 147.94 75.84) (end 152.2 75.84) (width 1) (layer "B.Cu") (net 2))
 (segment (start 196.695 69.495) (end 157.695 69.495) (width 1) (layer "B.Cu") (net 2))
 (segment (start 152.2 65.68) (end 153.88 65.68) (width 1) (layer "B.Cu") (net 2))
 (segment (start 152.2 101.24) (end 154.06 101.24) (width 1) (layer "B.Cu") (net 2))
 (segment (start 139.84 107.5) (end 139.8 107.5) (width 1) (layer "B.Cu") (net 2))
 (segment (start 152.2 83.46) (end 153.86 83.46) (width 1) (layer "B.Cu") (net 2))
 (segment (start 203 100.4) (end 198.2 105.2) (width 1) (layer "B.Cu") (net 2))
 (segment (start 153.88 65.68) (end 155.1 66.9) (width 1) (layer "B.Cu") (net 2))
 (segment (start 154.1 110.7) (end 154.9 109.9) (width 1) (layer "B.Cu") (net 2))
 (segment (start 184.4 105.2) (end 181.96 107.64) (width 1) (layer "B.Cu") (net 2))
 (segment (start 147.94 65.68) (end 152.2 65.68) (width 1) (layer "B.Cu") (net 2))
 (segment (start 154.84 75.84) (end 155.1 76.1) (width 1) (layer "B.Cu") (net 2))
 (segment (start 181.96 109.79) (end 179.42 109.79) (width 1) (layer "B.Cu") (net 2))
 (segment (start 139.8 107.5) (end 139.14 106.84) (width 1) (layer "B.Cu") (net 2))
 (segment (start 154.9 95) (end 153.74 96.16) (width 1) (layer "B.Cu") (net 2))
 (segment (start 157.695 69.495) (end 155.1 66.9) (width 1) (layer "B.Cu") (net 2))
 (segment (start 154.9 100.4) (end 154.9 95) (width 1) (layer "B.Cu") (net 2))
 (segment (start 139.14 70.78) (end 139.16 70.76) (width 1) (layer "B.Cu") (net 2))
 (segment (start 131.465 65.68) (end 133.75 67.965) (width 1) (layer "B.Cu") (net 2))
 (segment (start 198.2 105.2) (end 184.4 105.2) (width 1) (layer "B.Cu") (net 2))
 (segment (start 196.695 59.94) (end 196.695 69.495) (width 1) (layer "B.Cu") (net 2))
 (segment (start 141.2 108.86) (end 139.84 107.5) (width 1) (layer "B.Cu") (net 2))
 (segment (start 155.1 66.9) (end 155.1 76.1) (width 1) (layer "B.Cu") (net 2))
 (segment (start 139.92 80.92) (end 138.1 79.1) (width 1) (layer "F.Cu") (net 16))
 (segment (start 145.4 60.6) (end 143.3 60.6) (width 1) (layer "F.Cu") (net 16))
 (segment (start 151.75 56.5) (end 151 56.5) (width 1) (layer "F.Cu") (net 16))
 (segment (start 138.25 59.75) (end 136.5 58) (width 1) (layer "F.Cu") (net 16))
 (segment (start 141.2 80.92) (end 145.4 80.92) (width 1) (layer "F.Cu") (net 16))
 (segment (start 138.1 79.1) (end 138.1 68.5) (width 1) (layer "F.Cu") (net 16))
 (segment (start 139.1 60.6) (end 138.25 59.75) (width 1) (layer "F.Cu") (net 16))
 (segment (start 141.2 60.6) (end 139.1 60.6) (width 1) (layer "F.Cu") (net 16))
 (segment (start 136.5 58) (end 133.25 58) (width 1) (layer "F.Cu") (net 16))
 (segment (start 201.775 59.94) (end 201.775 58.025) (width 1) (layer "F.Cu") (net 16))
 (segment (start 200.25 56.5) (end 151.75 56.5) (width 1) (layer "F.Cu") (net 16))
 (segment (start 141.2 80.92) (end 139.92 80.92) (width 1) (layer "F.Cu") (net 16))
 (segment (start 201.775 58.025) (end 201.25 57.5) (width 1) (layer "F.Cu") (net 16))
 (segment (start 201.25 57.5) (end 200.25 56.5) (width 1) (layer "F.Cu") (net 16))
 (segment (start 143.3 60.6) (end 141.2 60.6) (width 1) (layer "F.Cu") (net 16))
 (via (at 138.25 59.75) (size 0.8) (drill 0.4) (layers "F.Cu" "B.Cu") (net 16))
 (via (at 138.1 68.5) (size 0.8) (drill 0.4) (layers "F.Cu" "B.Cu") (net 16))
 (via (at 133.25 58) (size 0.8) (drill 0.4) (layers "F.Cu" "B.Cu") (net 16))
 (via (at 151 56.5) (size 0.8) (drill 0.4) (layers "F.Cu" "B.Cu") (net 16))
 (segment (start 138.1 68.5) (end 138.1 59.9) (width 1) (layer "B.Cu") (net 16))
 (segment (start 128.925 59.075) (end 130 58) (width 1) (layer "B.Cu") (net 16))
 (segment (start 138.1 59.9) (end 138.25 59.75) (width 1) (layer "B.Cu") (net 16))
 (segment (start 151 56.5) (end 147.25 56.5) (width 1) (layer "B.Cu") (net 16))
 (segment (start 128.925 60.6) (end 128.925 59.075) (width 1) (layer "B.Cu") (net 16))
 (segment (start 147.25 56.5) (end 145.4 58.35) (width 1) (layer "B.Cu") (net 16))
 (segment (start 145.4 58.35) (end 145.4 60.6) (width 1) (layer "B.Cu") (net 16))
 (segment (start 133.25 58) (end 130 58) (width 1) (layer "B.Cu") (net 16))
 (segment (start 138.82 65.68) (end 141.2 65.68) (width 0.5) (layer "F.Cu") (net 18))
 (segment (start 135.25 67) (end 133.4005 68.8495) (width 0.5) (layer "F.Cu") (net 18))
 (segment (start 138.82 65.68) (end 136.57 65.68) (width 0.5) (layer "F.Cu") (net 18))
 (segment (start 168.75 69.047918) (end 158.351394 58.649312) (width 0.5) (layer "F.Cu") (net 18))
 (segment (start 133.4005 68.8495) (end 132.74005 68.8495) (width 0.5) (layer "F.Cu") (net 18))
 (segment (start 168.755 70.005) (end 168.75 70) (width 0.5) (layer "F.Cu") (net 18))
 (segment (start 136.57 65.68) (end 135.25 67) (width 0.5) (layer "F.Cu") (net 18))
 (segment (start 158.351394 58.649312) (end 158.350688 58.649312) (width 0.5) (layer "F.Cu") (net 18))
 (segment (start 168.75 70) (end 168.75 69.047918) (width 0.5) (layer "F.Cu") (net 18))
 (segment (start 168.755 80.26) (end 168.755 70.005) (width 0.5) (layer "F.Cu") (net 18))
 (segment (start 145.4 65.68) (end 141.2 65.68) (width 0.5) (layer "F.Cu") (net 18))
 (via (at 158.350688 58.649312) (size 0.8) (drill 0.4) (layers "F.Cu" "B.Cu") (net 18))
 (via (at 132.74005 68.8495) (size 0.8) (drill 0.4) (layers "F.Cu" "B.Cu") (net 18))
 (segment (start 145.9 54.85) (end 154.551376 54.85) (width 0.5) (layer "B.Cu") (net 18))
 (segment (start 132.0945 68.8495) (end 128.925 65.68) (width 0.5) (layer "B.Cu") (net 18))
 (segment (start 143.4 63.68) (end 143.4 57.35) (width 0.5) (layer "B.Cu") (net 18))
 (segment (start 145.4 65.68) (end 143.4 63.68) (width 0.5) (layer "B.Cu") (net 18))
 (segment (start 143.4 57.35) (end 145.9 54.85) (width 0.5) (layer "B.Cu") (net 18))
 (segment (start 132.74005 68.8495) (end 132.0945 68.8495) (width 0.5) (layer "B.Cu") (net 18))
 (segment (start 154.551376 54.85) (end 158.350688 58.649312) (width 0.5) (layer "B.Cu") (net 18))
 (segment (start 127.36 63.14) (end 126.75 63.75) (width 0.5) (layer "F.Cu") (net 17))
 (segment (start 127.5 68) (end 133.03 68) (width 0.5) (layer "F.Cu") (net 17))
 (segment (start 145.4 63.14) (end 141.2 63.14) (width 0.5) (layer "F.Cu") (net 17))
 (segment (start 126.75 67.25) (end 127.5 68) (width 0.5) (layer "F.Cu") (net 17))
 (segment (start 166.25 67.75) (end 159 60.5) (width 0.5) (layer "F.Cu") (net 17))
 (segment (start 126.75 63.75) (end 126.75 67.25) (width 0.5) (layer "F.Cu") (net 17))
 (segment (start 128.925 63.14) (end 127.36 63.14) (width 0.5) (layer "F.Cu") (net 17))
 (segment (start 166.215 67.785) (end 166.25 67.75) (width 0.5) (layer "F.Cu") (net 17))
 (segment (start 133.03 68) (end 137.89 63.14) (width 0.5) (layer "F.Cu") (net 17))
 (segment (start 141.2 63.14) (end 137.89 63.14) (width 0.5) (layer "F.Cu") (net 17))
 (segment (start 166.215 80.26) (end 166.215 67.785) (width 0.5) (layer "F.Cu") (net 17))
 (via (at 159 60.5) (size 0.8) (drill 0.4) (layers "F.Cu" "B.Cu") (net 17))
 (segment (start 154.05 55.55) (end 159 60.5) (width 0.5) (layer "B.Cu") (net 17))
 (segment (start 145.4 63.14) (end 144.1 61.84) (width 0.5) (layer "B.Cu") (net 17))
 (segment (start 144.1 61.84) (end 144.1 57.65) (width 0.5) (layer "B.Cu") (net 17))
 (segment (start 146.2 55.55) (end 154.05 55.55) (width 0.5) (layer "B.Cu") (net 17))
 (segment (start 144.1 57.65) (end 146.2 55.55) (width 0.5) (layer "B.Cu") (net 17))
 (segment (start 141.2 68.22) (end 145.4 68.22) (width 0.5) (layer "F.Cu") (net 21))
 (segment (start 147.94 68.22) (end 152.2 68.22) (width 0.5) (layer "F.Cu") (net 3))
 (segment (start 147.94 70.76) (end 152.2 70.76) (width 0.5) (layer "F.Cu") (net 4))
 (segment (start 141.2 73.3) (end 145.4 73.3) (width 0.5) (layer "F.Cu") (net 22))
 (segment (start 147.94 73.3) (end 152.2 73.3) (width 0.5) (layer "F.Cu") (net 5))
 (segment (start 141.2 75.84) (end 145.4 75.84) (width 0.5) (layer "F.Cu") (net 23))
 (segment (start 141.2 78.38) (end 145.4 78.38) (width 0.5) (layer "F.Cu") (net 24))
 (segment (start 147.94 78.38) (end 152.2 78.38) (width 0.5) (layer "F.Cu") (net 6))
 (segment (start 147.94 80.92) (end 152.2 80.92) (width 0.5) (layer "F.Cu") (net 7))
 (segment (start 141.2 83.46) (end 145.4 83.46) (width 0.5) (layer "F.Cu") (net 25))
 (segment (start 141.2 86) (end 145.4 86) (width 0.5) (layer "F.Cu") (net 26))
 (segment (start 147.94 86) (end 152.2 86) (width 0.5) (layer "F.Cu") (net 8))
 (segment (start 141.2 88.54) (end 145.4 88.54) (width 0.5) (layer "F.Cu") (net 27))
 (segment (start 147.94 88.54) (end 152.2 88.54) (width 0.5) (layer "F.Cu") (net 9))
 (segment (start 147.94 91.08) (end 152.2 91.08) (width 0.5) (layer "F.Cu") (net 10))
 (segment (start 141.2 93.62) (end 145.4 93.62) (width 0.5) (layer "F.Cu") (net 28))
 (segment (start 147.94 93.62) (end 152.2 93.62) (width 0.5) (layer "F.Cu") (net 11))
 (segment (start 141.2 96.16) (end 145.4 96.16) (width 0.5) (layer "F.Cu") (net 29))
 (segment (start 141.2 98.7) (end 145.4 98.7) (width 0.5) (layer "F.Cu") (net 30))
 (segment (start 147.94 98.7) (end 152.2 98.7) (width 0.5) (layer "F.Cu") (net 12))
 (segment (start 145.4 101.24) (end 141.2 101.24) (width 0.5) (layer "F.Cu") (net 31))
 (segment (start 145.4 103.78) (end 141.2 103.78) (width 0.5) (layer "F.Cu") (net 32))
 (segment (start 147.94 103.78) (end 152.2 103.78) (width 0.5) (layer "F.Cu") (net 13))
 (segment (start 145.4 106.32) (end 141.2 106.32) (width 0.5) (layer "F.Cu") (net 33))
 (segment (start 147.94 106.32) (end 152.2 106.32) (width 0.5) (layer "F.Cu") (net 14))
 (segment (start 147.94 108.86) (end 152.2 108.86) (width 0.5) (layer "F.Cu") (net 15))
 (segment (start 197.92 88) (end 197.92 98) (width 1) (layer "F.Cu") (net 19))
 (segment (start 187.04 107.26) (end 190.2 104.1) (width 1) (layer "F.Cu") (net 19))
 (segment (start 196 104.1) (end 197.92 102.18) (width 1) (layer "F.Cu") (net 19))
 (segment (start 190.2 104.1) (end 196 104.1) (width 1) (layer "F.Cu") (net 19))
 (segment (start 197.92 102.18) (end 197.92 98) (width 1) (layer "F.Cu") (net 19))
 (segment (start 187.04 109.79) (end 187.04 107.26) (width 1) (layer "F.Cu") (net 19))
 (segment (start 169.5 116) (end 170.75 116) (width 1) (layer "F.Cu") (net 20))
 (segment (start 130.06 112.81) (end 133.25 116) (width 1.5) (layer "F.Cu") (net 20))
 (segment (start 174.34 113.66) (end 172 116) (width 1.5) (layer "F.Cu") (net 20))
 (segment (start 133.25 116) (end 170.75 116) (width 1.5) (layer "F.Cu") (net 20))
 (segment (start 170.75 116) (end 172 116) (width 1) (layer "F.Cu") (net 20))
 (segment (start 172 116) (end 168.25 116) (width 1.5) (layer "F.Cu") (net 20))
 (segment (start 130.06 92.7) (end 130.06 112.81) (width 1.5) (layer "F.Cu") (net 20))
 (segment (start 174.34 109.79) (end 174.34 113.66) (width 1.5) (layer "F.Cu") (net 20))
 (segment (start 132.75 116) (end 168.25 116) (width 1) (layer "F.Cu") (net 20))
 (segment (start 168.25 116) (end 169.5 116) (width 1) (layer "F.Cu") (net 20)))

